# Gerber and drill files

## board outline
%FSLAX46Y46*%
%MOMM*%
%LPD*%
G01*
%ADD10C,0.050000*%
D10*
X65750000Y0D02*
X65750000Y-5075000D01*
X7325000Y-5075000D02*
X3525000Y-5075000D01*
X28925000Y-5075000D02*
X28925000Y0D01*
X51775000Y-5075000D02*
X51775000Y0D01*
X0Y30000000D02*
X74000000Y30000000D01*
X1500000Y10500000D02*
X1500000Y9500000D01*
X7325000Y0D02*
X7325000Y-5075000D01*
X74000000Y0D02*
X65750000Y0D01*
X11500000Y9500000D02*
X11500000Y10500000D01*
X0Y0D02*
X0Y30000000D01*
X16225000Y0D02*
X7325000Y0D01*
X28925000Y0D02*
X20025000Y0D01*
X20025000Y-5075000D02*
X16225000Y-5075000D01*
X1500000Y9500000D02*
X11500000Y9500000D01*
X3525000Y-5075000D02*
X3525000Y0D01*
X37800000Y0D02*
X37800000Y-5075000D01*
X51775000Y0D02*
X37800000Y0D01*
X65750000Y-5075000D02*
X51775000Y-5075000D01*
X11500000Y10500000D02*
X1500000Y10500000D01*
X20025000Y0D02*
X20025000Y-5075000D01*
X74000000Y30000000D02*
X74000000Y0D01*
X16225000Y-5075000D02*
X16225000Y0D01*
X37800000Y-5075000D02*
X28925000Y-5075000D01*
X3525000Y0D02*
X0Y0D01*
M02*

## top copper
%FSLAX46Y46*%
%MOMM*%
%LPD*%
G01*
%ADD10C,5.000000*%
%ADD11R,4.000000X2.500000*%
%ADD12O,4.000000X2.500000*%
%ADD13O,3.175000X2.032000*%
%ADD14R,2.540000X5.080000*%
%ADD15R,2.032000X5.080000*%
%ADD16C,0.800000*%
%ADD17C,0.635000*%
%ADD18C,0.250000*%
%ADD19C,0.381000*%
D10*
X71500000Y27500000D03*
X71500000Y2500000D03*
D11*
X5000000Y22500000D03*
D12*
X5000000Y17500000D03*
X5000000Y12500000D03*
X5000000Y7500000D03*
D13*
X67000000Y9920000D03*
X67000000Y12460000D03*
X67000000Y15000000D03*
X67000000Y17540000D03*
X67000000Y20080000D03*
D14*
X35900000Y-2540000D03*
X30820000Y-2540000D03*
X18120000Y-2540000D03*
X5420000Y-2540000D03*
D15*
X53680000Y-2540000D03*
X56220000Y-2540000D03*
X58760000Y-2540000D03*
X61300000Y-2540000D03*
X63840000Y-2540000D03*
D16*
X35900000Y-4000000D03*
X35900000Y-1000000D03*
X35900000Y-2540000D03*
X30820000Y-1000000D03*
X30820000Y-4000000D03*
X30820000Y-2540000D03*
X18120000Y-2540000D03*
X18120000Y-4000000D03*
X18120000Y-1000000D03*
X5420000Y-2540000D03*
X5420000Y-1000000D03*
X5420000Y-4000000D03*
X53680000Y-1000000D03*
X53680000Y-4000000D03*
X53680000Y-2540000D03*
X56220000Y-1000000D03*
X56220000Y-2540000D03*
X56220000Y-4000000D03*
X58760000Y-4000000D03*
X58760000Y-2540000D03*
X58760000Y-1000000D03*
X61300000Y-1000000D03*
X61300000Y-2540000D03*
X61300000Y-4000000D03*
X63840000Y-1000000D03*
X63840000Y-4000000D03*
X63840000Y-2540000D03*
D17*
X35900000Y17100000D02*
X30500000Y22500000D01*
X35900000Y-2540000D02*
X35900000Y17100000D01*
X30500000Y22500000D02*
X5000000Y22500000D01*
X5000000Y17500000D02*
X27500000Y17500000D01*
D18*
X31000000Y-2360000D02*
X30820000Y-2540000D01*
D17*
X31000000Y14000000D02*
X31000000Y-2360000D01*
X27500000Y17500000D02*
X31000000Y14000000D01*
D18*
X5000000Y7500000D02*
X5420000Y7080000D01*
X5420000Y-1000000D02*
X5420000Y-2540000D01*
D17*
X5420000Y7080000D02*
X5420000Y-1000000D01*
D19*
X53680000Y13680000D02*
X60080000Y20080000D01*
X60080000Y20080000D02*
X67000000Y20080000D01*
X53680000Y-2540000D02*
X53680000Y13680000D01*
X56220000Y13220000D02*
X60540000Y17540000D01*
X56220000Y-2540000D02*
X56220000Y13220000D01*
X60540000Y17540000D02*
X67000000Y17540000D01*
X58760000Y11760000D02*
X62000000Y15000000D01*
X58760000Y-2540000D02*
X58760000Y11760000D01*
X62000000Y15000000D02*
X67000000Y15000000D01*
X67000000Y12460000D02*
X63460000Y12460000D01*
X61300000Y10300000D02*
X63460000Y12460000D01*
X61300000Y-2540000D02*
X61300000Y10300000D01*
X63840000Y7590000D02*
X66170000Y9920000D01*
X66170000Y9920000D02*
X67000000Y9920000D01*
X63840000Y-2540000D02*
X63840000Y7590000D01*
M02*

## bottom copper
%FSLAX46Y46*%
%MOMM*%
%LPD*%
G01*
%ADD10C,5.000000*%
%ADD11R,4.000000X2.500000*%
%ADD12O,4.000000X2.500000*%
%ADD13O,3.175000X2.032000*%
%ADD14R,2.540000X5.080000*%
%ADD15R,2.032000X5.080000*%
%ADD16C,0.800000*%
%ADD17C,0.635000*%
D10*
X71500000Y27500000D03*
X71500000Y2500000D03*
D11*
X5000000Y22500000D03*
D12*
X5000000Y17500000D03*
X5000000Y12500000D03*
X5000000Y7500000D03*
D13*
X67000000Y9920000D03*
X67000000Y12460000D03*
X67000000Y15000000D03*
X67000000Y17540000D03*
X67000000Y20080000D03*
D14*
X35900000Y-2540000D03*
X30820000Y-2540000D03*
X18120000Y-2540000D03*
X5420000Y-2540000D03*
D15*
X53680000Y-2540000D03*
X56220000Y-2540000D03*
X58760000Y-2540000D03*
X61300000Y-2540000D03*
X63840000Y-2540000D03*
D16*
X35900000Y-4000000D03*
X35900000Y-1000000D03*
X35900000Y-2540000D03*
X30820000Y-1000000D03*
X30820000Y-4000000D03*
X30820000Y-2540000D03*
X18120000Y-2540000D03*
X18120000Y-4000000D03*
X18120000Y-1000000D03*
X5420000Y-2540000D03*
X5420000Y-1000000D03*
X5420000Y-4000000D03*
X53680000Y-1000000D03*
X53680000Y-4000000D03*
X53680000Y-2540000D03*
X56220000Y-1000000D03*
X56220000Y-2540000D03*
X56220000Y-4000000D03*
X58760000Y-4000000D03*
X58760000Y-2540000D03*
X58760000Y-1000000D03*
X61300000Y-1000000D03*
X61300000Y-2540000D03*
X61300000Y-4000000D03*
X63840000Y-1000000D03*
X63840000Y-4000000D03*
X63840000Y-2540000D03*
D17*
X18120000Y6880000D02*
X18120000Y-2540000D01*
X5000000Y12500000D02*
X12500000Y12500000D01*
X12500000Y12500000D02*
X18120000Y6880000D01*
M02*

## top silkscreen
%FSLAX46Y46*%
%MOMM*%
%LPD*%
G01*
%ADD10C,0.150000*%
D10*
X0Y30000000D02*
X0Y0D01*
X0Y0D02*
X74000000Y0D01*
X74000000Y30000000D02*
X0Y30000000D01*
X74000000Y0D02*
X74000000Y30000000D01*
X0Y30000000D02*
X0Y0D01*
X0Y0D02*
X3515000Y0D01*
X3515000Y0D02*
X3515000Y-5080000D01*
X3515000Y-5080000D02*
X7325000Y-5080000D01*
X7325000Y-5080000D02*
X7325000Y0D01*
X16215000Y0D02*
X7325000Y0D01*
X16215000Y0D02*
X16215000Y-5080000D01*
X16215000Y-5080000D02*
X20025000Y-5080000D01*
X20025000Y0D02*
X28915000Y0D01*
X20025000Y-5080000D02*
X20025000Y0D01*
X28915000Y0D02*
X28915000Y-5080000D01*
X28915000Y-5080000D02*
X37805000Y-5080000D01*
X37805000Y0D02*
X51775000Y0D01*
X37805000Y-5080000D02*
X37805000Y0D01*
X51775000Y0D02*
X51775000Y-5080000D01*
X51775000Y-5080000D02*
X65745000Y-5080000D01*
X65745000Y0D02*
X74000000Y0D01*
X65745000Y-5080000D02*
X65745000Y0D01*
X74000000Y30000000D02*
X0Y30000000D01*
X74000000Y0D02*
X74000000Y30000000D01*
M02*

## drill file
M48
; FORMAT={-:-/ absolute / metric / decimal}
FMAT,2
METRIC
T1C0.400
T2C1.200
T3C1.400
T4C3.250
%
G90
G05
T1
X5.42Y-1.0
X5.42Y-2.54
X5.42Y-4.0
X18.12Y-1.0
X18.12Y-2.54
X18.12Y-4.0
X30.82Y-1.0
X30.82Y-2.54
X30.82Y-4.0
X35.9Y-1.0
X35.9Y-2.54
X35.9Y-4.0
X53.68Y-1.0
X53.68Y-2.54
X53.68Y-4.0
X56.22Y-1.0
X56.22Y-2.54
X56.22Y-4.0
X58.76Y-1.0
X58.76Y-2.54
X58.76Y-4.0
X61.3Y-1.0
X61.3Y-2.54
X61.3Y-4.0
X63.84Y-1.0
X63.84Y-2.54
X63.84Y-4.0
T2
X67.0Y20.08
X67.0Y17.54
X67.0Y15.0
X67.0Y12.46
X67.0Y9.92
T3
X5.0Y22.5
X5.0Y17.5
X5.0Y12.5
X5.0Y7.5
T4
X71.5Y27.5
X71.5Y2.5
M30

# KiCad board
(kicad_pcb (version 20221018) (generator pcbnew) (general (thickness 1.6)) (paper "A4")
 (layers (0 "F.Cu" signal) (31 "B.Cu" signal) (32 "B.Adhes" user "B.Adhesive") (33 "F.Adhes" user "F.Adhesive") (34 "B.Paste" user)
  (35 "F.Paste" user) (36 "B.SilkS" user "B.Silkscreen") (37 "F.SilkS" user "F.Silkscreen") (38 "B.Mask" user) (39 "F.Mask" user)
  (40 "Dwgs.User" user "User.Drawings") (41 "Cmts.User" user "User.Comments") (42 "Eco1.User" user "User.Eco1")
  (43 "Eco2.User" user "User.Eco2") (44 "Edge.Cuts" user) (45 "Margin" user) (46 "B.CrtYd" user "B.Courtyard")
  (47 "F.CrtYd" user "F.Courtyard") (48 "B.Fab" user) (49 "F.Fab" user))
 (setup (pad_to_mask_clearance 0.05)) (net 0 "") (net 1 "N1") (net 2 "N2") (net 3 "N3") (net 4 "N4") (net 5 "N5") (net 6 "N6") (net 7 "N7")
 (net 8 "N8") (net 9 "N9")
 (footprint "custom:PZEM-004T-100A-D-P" (layer "F.Cu") (at 0 0)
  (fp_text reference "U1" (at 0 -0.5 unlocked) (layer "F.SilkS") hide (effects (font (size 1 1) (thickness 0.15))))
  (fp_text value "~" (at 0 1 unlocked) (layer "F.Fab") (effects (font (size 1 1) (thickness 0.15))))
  (fp_line (start 0 -30) (end 0 0) (stroke (width 0.15) (type default)) (layer "F.SilkS"))
  (fp_line (start 0 0) (end 74 0) (stroke (width 0.15) (type default)) (layer "F.SilkS"))
  (fp_line (start 74 -30) (end 0 -30) (stroke (width 0.15) (type default)) (layer "F.SilkS"))
  (fp_line (start 74 0) (end 74 -30) (stroke (width 0.15) (type default)) (layer "F.SilkS"))
  (pad "" thru_hole circle (at 71.5 -27.5) (size 5 5) (drill 3.25) (layers "*.Cu" "*.Mask"))
  (pad "" thru_hole circle (at 71.5 -2.5) (size 5 5) (drill 3.25) (layers "*.Cu" "*.Mask"))
  (pad "1" thru_hole rect (at 5 -22.5) (size 4 2.5) (drill 1.4) (layers "*.Cu" "*.Mask") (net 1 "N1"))
  (pad "2" thru_hole oval (at 5 -17.5) (size 4 2.5) (drill 1.4) (layers "*.Cu" "*.Mask") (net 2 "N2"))
  (pad "3" thru_hole oval (at 5 -12.5) (size 4 2.5) (drill 1.4) (layers "*.Cu" "*.Mask") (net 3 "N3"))
  (pad "4" thru_hole oval (at 5 -7.5) (size 4 2.5) (drill 1.4) (layers "*.Cu" "*.Mask") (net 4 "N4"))
  (pad "5" thru_hole oval (at 67 -9.92) (size 3.175 2.032) (drill 1.2) (layers "*.Cu" "*.Mask") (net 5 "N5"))
  (pad "6" thru_hole oval (at 67 -12.46) (size 3.175 2.032) (drill 1.2) (layers "*.Cu" "*.Mask") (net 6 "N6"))
  (pad "7" thru_hole oval (at 67 -15) (size 3.175 2.032) (drill 1.2) (layers "*.Cu" "*.Mask") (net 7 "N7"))
  (pad "8" thru_hole oval (at 67 -17.54) (size 3.175 2.032) (drill 1.2) (layers "*.Cu" "*.Mask") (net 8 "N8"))
  (pad "9" thru_hole oval (at 67 -20.08) (size 3.175 2.032) (drill 1.2) (layers "*.Cu" "*.Mask") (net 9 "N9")))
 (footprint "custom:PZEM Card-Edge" (layer "F.Cu") (at 0 0)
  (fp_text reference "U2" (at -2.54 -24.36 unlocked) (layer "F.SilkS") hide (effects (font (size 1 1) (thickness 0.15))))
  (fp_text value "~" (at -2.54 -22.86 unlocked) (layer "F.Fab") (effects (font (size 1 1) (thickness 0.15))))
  (fp_line (start 0 -30) (end 0 0) (stroke (width 0.15) (type default)) (layer "F.SilkS"))
  (fp_line (start 0 0) (end 3.515 0) (stroke (width 0.15) (type default)) (layer "F.SilkS"))
  (fp_line (start 3.515 0) (end 3.515 5.08) (stroke (width 0.15) (type default)) (layer "F.SilkS"))
  (fp_line (start 3.515 5.08) (end 7.325 5.08) (stroke (width 0.15) (type default)) (layer "F.SilkS"))
  (fp_line (start 7.325 5.08) (end 7.325 0) (stroke (width 0.15) (type default)) (layer "F.SilkS"))
  (fp_line (start 16.215 0) (end 7.325 0) (stroke (width 0.15) (type default)) (layer "F.SilkS"))
  (fp_line (start 16.215 0) (end 16.215 5.08) (stroke (width 0.15) (type default)) (layer "F.SilkS"))
  (fp_line (start 16.215 5.08) (end 20.025 5.08) (stroke (width 0.15) (type default)) (layer "F.SilkS"))
  (fp_line (start 20.025 0) (end 28.915 0) (stroke (width 0.15) (type default)) (layer "F.SilkS"))
  (fp_line (start 20.025 5.08) (end 20.025 0) (stroke (width 0.15) (type default)) (layer "F.SilkS"))
  (fp_line (start 28.915 0) (end 28.915 5.08) (stroke (width 0.15) (type default)) (layer "F.SilkS"))
  (fp_line (start 28.915 5.08) (end 37.805 5.08) (stroke (width 0.15) (type default)) (layer "F.SilkS"))
  (fp_line (start 37.805 0) (end 51.775 0) (stroke (width 0.15) (type default)) (layer "F.SilkS"))
  (fp_line (start 37.805 5.08) (end 37.805 0) (stroke (width 0.15) (type default)) (layer "F.SilkS"))
  (fp_line (start 51.775 0) (end 51.775 5.08) (stroke (width 0.15) (type default)) (layer "F.SilkS"))
  (fp_line (start 51.775 5.08) (end 65.745 5.08) (stroke (width 0.15) (type default)) (layer "F.SilkS"))
  (fp_line (start 65.745 0) (end 74 0) (stroke (width 0.15) (type default)) (layer "F.SilkS"))
  (fp_line (start 65.745 5.08) (end 65.745 0) (stroke (width 0.15) (type default)) (layer "F.SilkS"))
  (fp_line (start 74 -30) (end 0 -30) (stroke (width 0.15) (type default)) (layer "F.SilkS"))
  (fp_line (start 74 0) (end 74 -30) (stroke (width 0.15) (type default)) (layer "F.SilkS"))
  (pad "1" connect rect (at 35.9 2.54 90) (size 5.08 2.54) (layers "F.Cu" "F.Mask") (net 1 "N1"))
  (pad "1" connect rect (at 35.9 2.54 90) (size 5.08 2.54) (layers "B.Cu" "B.Mask") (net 1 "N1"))
  (pad "2" connect rect (at 30.82 2.54 90) (size 5.08 2.54) (layers "F.Cu" "F.Mask") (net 2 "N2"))
  (pad "2" connect rect (at 30.82 2.54 90) (size 5.08 2.54) (layers "B.Cu" "B.Mask") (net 2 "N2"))
  (pad "3" connect rect (at 18.12 2.54 90) (size 5.08 2.54) (layers "F.Cu" "F.Mask") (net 3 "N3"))
  (pad "3" connect rect (at 18.12 2.54 90) (size 5.08 2.54) (layers "B.Cu" "B.Mask") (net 3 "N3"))
  (pad "4" connect rect (at 5.42 2.54 90) (size 5.08 2.54) (layers "F.Cu" "F.Mask") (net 4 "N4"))
  (pad "4" connect rect (at 5.42 2.54 90) (size 5.08 2.54) (layers "B.Cu" "B.Mask") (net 4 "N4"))
  (pad "5" connect rect (at 53.68 2.54 270) (size 5.08 2.032) (layers "F.Cu" "F.Mask") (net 5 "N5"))
  (pad "5" connect rect (at 53.68 2.54 270) (size 5.08 2.032) (layers "B.Cu" "B.Mask") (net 5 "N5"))
  (pad "6" connect rect (at 56.22 2.54 270) (size 5.08 2.032) (layers "F.Cu" "F.Mask") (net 6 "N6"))
  (pad "6" connect rect (at 56.22 2.54 270) (size 5.08 2.032) (layers "B.Cu" "B.Mask") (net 6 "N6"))
  (pad "7" connect rect (at 58.76 2.54 270) (size 5.08 2.032) (layers "F.Cu" "F.Mask") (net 7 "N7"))
  (pad "7" connect rect (at 58.76 2.54 270) (size 5.08 2.032) (layers "B.Cu" "B.Mask") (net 7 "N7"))
  (pad "8" connect rect (at 61.3 2.54 270) (size 5.08 2.032) (layers "F.Cu" "F.Mask") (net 8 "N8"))
  (pad "8" connect rect (at 61.3 2.54 270) (size 5.08 2.032) (layers "B.Cu" "B.Mask") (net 8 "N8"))
  (pad "9" connect rect (at 63.84 2.54 270) (size 5.08 2.032) (layers "F.Cu" "F.Mask") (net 9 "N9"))
  (pad "9" connect rect (at 63.84 2.54 270) (size 5.08 2.032) (layers "B.Cu" "B.Mask") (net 9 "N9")))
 (gr_line (start 65.75 0) (end 65.75 5.075) (stroke (width 0.05) (type default)) (layer "Edge.Cuts"))
 (gr_line (start 7.325 5.075) (end 3.525 5.075) (stroke (width 0.05) (type default)) (layer "Edge.Cuts"))
 (gr_line (start 28.925 5.075) (end 28.925 0) (stroke (width 0.05) (type default)) (layer "Edge.Cuts"))
 (gr_line (start 51.775 5.075) (end 51.775 0) (stroke (width 0.05) (type default)) (layer "Edge.Cuts"))
 (gr_line (start 0 -30) (end 74 -30) (stroke (width 0.05) (type default)) (layer "Edge.Cuts"))
 (gr_line (start 1.5 -10.5) (end 1.5 -9.5) (stroke (width 0.05) (type default)) (layer "Edge.Cuts"))
 (gr_line (start 7.325 0) (end 7.325 5.075) (stroke (width 0.05) (type default)) (layer "Edge.Cuts"))
 (gr_line (start 74 0) (end 65.75 0) (stroke (width 0.05) (type default)) (layer "Edge.Cuts"))
 (gr_line (start 11.5 -9.5) (end 11.5 -10.5) (stroke (width 0.05) (type default)) (layer "Edge.Cuts"))
 (gr_line (start 0 0) (end 0 -30) (stroke (width 0.05) (type default)) (layer "Edge.Cuts"))
 (gr_line (start 16.225 0) (end 7.325 0) (stroke (width 0.05) (type default)) (layer "Edge.Cuts"))
 (gr_line (start 28.925 0) (end 20.025 0) (stroke (width 0.05) (type default)) (layer "Edge.Cuts"))
 (gr_line (start 20.025 5.075) (end 16.225 5.075) (stroke (width 0.05) (type default)) (layer "Edge.Cuts"))
 (gr_line (start 1.5 -9.5) (end 11.5 -9.5) (stroke (width 0.05) (type default)) (layer "Edge.Cuts"))
 (gr_line (start 3.525 5.075) (end 3.525 0) (stroke (width 0.05) (type default)) (layer "Edge.Cuts"))
 (gr_line (start 37.8 0) (end 37.8 5.075) (stroke (width 0.05) (type default)) (layer "Edge.Cuts"))
 (gr_line (start 51.775 0) (end 37.8 0) (stroke (width 0.05) (type default)) (layer "Edge.Cuts"))
 (gr_line (start 65.75 5.075) (end 51.775 5.075) (stroke (width 0.05) (type default)) (layer "Edge.Cuts"))
 (gr_line (start 11.5 -10.5) (end 1.5 -10.5) (stroke (width 0.05) (type default)) (layer "Edge.Cuts"))
 (gr_line (start 20.025 0) (end 20.025 5.075) (stroke (width 0.05) (type default)) (layer "Edge.Cuts"))
 (gr_line (start 74 -30) (end 74 0) (stroke (width 0.05) (type default)) (layer "Edge.Cuts"))
 (gr_line (start 16.225 5.075) (end 16.225 0) (stroke (width 0.05) (type default)) (layer "Edge.Cuts"))
 (gr_line (start 37.8 5.075) (end 28.925 5.075) (stroke (width 0.05) (type default)) (layer "Edge.Cuts"))
 (gr_line (start 3.525 0) (end 0 0) (stroke (width 0.05) (type default)) (layer "Edge.Cuts"))
 (segment (start 35.9 -17.1) (end 30.5 -22.5) (width 0.635) (layer "F.Cu") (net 1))
 (segment (start 35.9 2.54) (end 35.9 -17.1) (width 0.635) (layer "F.Cu") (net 1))
 (segment (start 30.5 -22.5) (end 5 -22.5) (width 0.635) (layer "F.Cu") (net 1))
 (via (at 35.9 4) (size 0.8) (drill 0.4) (layers "F.Cu" "B.Cu") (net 1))
 (via (at 35.9 1) (size 0.8) (drill 0.4) (layers "F.Cu" "B.Cu") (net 1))
 (via (at 35.9 2.54) (size 0.8) (drill 0.4) (layers "F.Cu" "B.Cu") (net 1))
 (segment (start 5 -17.5) (end 27.5 -17.5) (width 0.635) (layer "F.Cu") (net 2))
 (segment (start 31 2.36) (end 30.82 2.54) (width 0.25) (layer "F.Cu") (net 2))
 (segment (start 31 -14) (end 31 2.36) (width 0.635) (layer "F.Cu") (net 2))
 (segment (start 27.5 -17.5) (end 31 -14) (width 0.635) (layer "F.Cu") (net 2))
 (via (at 30.82 1) (size 0.8) (drill 0.4) (layers "F.Cu" "B.Cu") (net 2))
 (via (at 30.82 4) (size 0.8) (drill 0.4) (layers "F.Cu" "B.Cu") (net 2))
 (via (at 30.82 2.54) (size 0.8) (drill 0.4) (layers "F.Cu" "B.Cu") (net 2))
 (via (at 18.12 2.54) (size 0.8) (drill 0.4) (layers "F.Cu" "B.Cu") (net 3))
 (via (at 18.12 4) (size 0.8) (drill 0.4) (layers "F.Cu" "B.Cu") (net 3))
 (via (at 18.12 1) (size 0.8) (drill 0.4) (layers "F.Cu" "B.Cu") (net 3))
 (segment (start 18.12 -6.88) (end 18.12 2.54) (width 0.635) (layer "B.Cu") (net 3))
 (segment (start 5 -12.5) (end 12.5 -12.5) (width 0.635) (layer "B.Cu") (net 3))
 (segment (start 12.5 -12.5) (end 18.12 -6.88) (width 0.635) (layer "B.Cu") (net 3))
 (segment (start 5 -7.5) (end 5.42 -7.08) (width 0.25) (layer "F.Cu") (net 4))
 (segment (start 5.42 1) (end 5.42 2.54) (width 0.25) (layer "F.Cu") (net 4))
 (segment (start 5.42 -7.08) (end 5.42 1) (width 0.635) (layer "F.Cu") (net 4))
 (via (at 5.42 2.54) (size 0.8) (drill 0.4) (layers "F.Cu" "B.Cu") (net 4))
 (via (at 5.42 1) (size 0.8) (drill 0.4) (layers "F.Cu" "B.Cu") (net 4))
 (via (at 5.42 4) (size 0.8) (drill 0.4) (layers "F.Cu" "B.Cu") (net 4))
 (segment (start 53.68 -13.68) (end 60.08 -20.08) (width 0.381) (layer "F.Cu") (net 5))
 (segment (start 60.08 -20.08) (end 67 -20.08) (width 0.381) (layer "F.Cu") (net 5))
 (segment (start 53.68 2.54) (end 53.68 -13.68) (width 0.381) (layer "F.Cu") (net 5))
 (via (at 53.68 1) (size 0.8) (drill 0.4) (layers "F.Cu" "B.Cu") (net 5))
 (via (at 53.68 4) (size 0.8) (drill 0.4) (layers "F.Cu" "B.Cu") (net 5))
 (via (at 53.68 2.54) (size 0.8) (drill 0.4) (layers "F.Cu" "B.Cu") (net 5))
 (segment (start 56.22 -13.22) (end 60.54 -17.54) (width 0.381) (layer "F.Cu") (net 6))
 (segment (start 56.22 2.54) (end 56.22 -13.22) (width 0.381) (layer "F.Cu") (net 6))
 (segment (start 60.54 -17.54) (end 67 -17.54) (width 0.381) (layer "F.Cu") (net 6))
 (via (at 56.22 1) (size 0.8) (drill 0.4) (layers "F.Cu" "B.Cu") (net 6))
 (via (at 56.22 2.54) (size 0.8) (drill 0.4) (layers "F.Cu" "B.Cu") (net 6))
 (via (at 56.22 4) (size 0.8) (drill 0.4) (layers "F.Cu" "B.Cu") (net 6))
 (segment (start 58.76 -11.76) (end 62 -15) (width 0.381) (layer "F.Cu") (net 7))
 (segment (start 58.76 2.54) (end 58.76 -11.76) (width 0.381) (layer "F.Cu") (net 7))
 (segment (start 62 -15) (end 67 -15) (width 0.381) (layer "F.Cu") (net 7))
 (via (at 58.76 4) (size 0.8) (drill 0.4) (layers "F.Cu" "B.Cu") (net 7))
 (via (at 58.76 2.54) (size 0.8) (drill 0.4) (layers "F.Cu" "B.Cu") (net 7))
 (via (at 58.76 1) (size 0.8) (drill 0.4) (layers "F.Cu" "B.Cu") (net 7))
 (segment (start 67 -12.46) (end 63.46 -12.46) (width 0.381) (layer "F.Cu") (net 8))
 (segment (start 61.3 -10.3) (end 63.46 -12.46) (width 0.381) (layer "F.Cu") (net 8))
 (segment (start 61.3 2.54) (end 61.3 -10.3) (width 0.381) (layer "F.Cu") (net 8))
 (via (at 61.3 1) (size 0.8) (drill 0.4) (layers "F.Cu" "B.Cu") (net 8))
 (via (at 61.3 2.54) (size 0.8) (drill 0.4) (layers "F.Cu" "B.Cu") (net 8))
 (via (at 61.3 4) (size 0.8) (drill 0.4) (layers "F.Cu" "B.Cu") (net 8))
 (segment (start 63.84 -7.59) (end 66.17 -9.92) (width 0.381) (layer "F.Cu") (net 9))
 (segment (start 66.17 -9.92) (end 67 -9.92) (width 0.381) (layer "F.Cu") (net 9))
 (segment (start 63.84 2.54) (end 63.84 -7.59) (width 0.381) (layer "F.Cu") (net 9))
 (via (at 63.84 1) (size 0.8) (drill 0.4) (layers "F.Cu" "B.Cu") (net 9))
 (via (at 63.84 4) (size 0.8) (drill 0.4) (layers "F.Cu" "B.Cu") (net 9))
 (via (at 63.84 2.54) (size 0.8) (drill 0.4) (layers "F.Cu" "B.Cu") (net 9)))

